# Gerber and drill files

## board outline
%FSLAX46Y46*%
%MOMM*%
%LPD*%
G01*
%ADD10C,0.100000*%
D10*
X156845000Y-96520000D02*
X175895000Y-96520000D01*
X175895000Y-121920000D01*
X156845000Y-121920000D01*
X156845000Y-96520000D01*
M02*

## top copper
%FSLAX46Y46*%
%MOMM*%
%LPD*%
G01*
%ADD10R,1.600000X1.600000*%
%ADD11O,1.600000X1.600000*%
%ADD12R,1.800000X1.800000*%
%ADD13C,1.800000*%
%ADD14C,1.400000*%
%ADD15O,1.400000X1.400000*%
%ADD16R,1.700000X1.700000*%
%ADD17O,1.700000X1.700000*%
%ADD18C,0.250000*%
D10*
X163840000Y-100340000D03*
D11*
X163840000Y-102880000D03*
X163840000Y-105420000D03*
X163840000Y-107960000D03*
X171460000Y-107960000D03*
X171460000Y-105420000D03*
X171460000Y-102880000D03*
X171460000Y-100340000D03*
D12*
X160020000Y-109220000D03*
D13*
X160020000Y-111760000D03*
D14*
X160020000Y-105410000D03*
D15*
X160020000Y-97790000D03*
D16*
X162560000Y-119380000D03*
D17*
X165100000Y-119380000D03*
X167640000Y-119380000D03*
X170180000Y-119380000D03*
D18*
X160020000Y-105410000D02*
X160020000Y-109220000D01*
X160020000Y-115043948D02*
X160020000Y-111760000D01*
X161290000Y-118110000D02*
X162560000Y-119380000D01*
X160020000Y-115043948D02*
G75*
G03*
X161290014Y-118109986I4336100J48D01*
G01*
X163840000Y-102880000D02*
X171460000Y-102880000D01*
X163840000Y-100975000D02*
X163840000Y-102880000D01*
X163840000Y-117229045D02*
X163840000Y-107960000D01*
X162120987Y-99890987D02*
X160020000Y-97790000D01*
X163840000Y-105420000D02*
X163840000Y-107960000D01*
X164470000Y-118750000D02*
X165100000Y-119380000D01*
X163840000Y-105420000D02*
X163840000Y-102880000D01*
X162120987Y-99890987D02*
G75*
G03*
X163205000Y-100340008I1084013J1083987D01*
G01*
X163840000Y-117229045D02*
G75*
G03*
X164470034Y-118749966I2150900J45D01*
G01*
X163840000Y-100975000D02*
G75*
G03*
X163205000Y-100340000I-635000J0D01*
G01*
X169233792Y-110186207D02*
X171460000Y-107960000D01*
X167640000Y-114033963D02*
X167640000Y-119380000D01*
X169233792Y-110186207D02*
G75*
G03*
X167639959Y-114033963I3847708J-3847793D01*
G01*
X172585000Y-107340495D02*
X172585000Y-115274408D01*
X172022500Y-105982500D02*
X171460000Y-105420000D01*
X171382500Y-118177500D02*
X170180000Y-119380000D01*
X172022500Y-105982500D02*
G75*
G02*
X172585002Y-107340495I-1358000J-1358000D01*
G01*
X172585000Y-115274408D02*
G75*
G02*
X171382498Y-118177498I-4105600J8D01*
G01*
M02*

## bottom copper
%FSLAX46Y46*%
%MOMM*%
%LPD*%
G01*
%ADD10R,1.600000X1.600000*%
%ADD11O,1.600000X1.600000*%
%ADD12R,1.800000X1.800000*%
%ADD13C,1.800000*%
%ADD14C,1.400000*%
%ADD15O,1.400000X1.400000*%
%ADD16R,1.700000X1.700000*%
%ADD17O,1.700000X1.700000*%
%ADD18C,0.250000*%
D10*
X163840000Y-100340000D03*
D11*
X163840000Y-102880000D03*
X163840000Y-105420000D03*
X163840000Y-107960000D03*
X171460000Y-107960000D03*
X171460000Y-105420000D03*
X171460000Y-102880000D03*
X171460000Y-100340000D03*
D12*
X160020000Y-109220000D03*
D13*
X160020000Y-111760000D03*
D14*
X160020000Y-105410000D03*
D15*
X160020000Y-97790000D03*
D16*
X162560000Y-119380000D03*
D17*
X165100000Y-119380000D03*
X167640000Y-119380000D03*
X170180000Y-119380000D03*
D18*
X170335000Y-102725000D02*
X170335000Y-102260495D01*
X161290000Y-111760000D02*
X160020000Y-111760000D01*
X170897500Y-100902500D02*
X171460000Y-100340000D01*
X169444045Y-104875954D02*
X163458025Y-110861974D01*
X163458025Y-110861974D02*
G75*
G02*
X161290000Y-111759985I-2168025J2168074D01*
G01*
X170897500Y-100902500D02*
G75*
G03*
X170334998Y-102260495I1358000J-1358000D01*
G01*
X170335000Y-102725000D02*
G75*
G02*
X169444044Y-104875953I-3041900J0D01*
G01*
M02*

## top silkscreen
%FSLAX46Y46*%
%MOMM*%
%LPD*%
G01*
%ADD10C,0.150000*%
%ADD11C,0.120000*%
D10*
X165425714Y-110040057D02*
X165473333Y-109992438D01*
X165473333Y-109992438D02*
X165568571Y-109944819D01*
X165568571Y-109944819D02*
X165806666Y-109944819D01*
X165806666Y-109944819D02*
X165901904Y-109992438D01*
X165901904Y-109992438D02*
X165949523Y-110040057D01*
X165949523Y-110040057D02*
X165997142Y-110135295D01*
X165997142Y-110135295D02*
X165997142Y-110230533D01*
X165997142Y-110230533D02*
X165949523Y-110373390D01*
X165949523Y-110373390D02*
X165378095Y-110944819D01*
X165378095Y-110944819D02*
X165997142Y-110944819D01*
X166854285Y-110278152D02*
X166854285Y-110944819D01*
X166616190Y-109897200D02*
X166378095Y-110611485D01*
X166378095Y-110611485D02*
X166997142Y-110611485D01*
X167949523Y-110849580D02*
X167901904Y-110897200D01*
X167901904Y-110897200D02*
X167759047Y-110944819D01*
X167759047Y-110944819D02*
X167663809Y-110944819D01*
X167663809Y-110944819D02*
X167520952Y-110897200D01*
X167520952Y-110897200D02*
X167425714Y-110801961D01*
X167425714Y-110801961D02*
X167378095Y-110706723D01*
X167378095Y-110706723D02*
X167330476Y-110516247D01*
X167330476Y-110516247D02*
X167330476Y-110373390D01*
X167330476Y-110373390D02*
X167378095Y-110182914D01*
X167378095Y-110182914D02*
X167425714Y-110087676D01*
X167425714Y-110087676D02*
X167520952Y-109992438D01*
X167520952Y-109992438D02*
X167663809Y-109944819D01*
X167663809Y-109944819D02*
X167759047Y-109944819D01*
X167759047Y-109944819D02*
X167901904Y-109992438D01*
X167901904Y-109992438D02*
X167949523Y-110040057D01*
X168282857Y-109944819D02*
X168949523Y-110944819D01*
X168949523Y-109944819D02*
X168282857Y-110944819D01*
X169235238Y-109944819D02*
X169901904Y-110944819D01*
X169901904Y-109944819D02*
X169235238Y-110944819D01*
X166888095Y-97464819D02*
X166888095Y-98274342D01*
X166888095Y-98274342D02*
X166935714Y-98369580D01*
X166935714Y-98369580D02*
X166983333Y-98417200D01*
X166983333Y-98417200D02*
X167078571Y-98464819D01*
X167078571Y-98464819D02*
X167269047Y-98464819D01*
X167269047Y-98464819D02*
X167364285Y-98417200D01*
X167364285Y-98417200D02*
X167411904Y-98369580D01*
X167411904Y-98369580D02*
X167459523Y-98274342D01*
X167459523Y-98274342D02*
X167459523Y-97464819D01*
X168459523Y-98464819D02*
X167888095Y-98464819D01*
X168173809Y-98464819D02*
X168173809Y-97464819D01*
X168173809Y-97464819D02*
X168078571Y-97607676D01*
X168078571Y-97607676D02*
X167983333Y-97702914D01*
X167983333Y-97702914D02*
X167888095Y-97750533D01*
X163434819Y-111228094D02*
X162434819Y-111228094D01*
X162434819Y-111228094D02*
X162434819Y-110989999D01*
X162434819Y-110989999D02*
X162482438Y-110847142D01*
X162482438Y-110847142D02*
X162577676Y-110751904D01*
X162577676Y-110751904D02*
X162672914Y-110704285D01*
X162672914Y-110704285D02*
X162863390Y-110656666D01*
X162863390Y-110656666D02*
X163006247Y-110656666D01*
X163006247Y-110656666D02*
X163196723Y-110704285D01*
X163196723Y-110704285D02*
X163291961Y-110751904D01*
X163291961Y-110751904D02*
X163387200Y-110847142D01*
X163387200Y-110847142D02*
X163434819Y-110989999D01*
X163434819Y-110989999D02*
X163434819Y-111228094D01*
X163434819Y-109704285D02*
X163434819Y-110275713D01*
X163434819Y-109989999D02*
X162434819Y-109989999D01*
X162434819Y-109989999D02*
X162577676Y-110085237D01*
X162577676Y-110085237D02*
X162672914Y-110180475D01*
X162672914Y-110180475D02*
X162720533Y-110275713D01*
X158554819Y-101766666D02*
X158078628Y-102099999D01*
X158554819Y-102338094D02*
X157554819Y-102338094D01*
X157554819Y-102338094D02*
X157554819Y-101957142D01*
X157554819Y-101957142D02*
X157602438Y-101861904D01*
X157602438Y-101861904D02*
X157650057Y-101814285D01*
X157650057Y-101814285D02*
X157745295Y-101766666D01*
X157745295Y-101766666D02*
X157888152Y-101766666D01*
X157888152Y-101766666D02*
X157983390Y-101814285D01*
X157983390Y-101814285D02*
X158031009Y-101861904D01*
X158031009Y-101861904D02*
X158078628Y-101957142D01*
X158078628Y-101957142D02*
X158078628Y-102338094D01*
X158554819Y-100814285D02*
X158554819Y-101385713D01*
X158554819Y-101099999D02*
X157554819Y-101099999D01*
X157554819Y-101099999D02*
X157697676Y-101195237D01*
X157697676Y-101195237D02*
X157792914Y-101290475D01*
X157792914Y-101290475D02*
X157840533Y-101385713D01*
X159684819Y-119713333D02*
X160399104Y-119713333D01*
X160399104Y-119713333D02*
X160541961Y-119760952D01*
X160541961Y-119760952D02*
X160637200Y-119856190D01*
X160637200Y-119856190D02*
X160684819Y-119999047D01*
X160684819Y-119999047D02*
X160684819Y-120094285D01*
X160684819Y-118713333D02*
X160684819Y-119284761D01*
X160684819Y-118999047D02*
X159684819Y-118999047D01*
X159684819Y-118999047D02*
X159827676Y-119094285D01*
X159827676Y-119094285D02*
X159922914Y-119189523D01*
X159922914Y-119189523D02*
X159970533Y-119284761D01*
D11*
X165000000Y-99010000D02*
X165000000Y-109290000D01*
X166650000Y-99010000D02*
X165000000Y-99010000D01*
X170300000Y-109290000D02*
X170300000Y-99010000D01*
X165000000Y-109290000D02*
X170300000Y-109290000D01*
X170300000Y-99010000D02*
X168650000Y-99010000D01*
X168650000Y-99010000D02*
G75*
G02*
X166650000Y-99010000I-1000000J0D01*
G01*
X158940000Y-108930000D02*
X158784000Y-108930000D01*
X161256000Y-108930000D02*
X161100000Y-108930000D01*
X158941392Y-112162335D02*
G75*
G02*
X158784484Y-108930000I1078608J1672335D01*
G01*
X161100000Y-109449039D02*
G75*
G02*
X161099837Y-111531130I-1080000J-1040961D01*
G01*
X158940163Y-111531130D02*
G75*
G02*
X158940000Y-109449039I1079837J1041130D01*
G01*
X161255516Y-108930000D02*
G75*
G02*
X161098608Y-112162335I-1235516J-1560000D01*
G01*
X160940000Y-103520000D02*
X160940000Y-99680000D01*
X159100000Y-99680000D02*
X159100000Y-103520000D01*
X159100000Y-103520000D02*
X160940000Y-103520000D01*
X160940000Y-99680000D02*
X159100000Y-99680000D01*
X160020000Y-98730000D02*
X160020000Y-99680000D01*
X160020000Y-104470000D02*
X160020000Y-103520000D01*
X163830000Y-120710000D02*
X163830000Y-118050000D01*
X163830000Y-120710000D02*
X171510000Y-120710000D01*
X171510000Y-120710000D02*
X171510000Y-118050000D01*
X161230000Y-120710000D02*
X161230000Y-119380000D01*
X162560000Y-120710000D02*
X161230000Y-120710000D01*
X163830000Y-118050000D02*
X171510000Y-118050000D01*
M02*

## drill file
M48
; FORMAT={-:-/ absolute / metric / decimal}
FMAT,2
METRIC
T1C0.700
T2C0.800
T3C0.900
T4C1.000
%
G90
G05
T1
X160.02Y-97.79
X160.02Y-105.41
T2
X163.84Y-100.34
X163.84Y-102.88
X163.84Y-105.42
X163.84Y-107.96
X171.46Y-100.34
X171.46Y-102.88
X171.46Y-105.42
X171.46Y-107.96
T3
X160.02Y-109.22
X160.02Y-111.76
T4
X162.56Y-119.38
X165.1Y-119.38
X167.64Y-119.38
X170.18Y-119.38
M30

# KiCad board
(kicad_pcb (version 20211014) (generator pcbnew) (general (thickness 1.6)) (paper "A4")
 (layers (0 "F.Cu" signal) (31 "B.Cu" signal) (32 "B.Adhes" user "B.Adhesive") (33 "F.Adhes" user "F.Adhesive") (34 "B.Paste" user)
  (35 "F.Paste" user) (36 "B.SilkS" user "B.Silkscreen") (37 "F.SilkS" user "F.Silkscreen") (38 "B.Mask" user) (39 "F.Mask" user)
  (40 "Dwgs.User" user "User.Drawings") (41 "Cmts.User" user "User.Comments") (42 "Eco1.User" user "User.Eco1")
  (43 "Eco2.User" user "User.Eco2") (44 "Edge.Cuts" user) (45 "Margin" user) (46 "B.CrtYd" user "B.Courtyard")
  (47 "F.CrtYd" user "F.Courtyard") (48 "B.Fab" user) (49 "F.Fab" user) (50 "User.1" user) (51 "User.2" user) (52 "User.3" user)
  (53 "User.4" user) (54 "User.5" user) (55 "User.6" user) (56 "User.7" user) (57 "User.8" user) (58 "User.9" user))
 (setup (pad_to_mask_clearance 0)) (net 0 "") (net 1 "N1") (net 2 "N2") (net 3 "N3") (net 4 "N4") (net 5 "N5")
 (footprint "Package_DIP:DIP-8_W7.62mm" (layer "F.Cu") (at 163.84 100.34)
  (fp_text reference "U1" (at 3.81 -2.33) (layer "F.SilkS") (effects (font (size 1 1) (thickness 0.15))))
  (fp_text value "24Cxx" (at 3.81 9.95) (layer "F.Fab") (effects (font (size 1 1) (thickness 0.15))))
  (fp_line (start 1.16 -1.33) (end 1.16 8.95) (layer "F.SilkS") (width 0.12))
  (fp_line (start 2.81 -1.33) (end 1.16 -1.33) (layer "F.SilkS") (width 0.12))
  (fp_line (start 6.46 8.95) (end 6.46 -1.33) (layer "F.SilkS") (width 0.12))
  (fp_line (start 1.16 8.95) (end 6.46 8.95) (layer "F.SilkS") (width 0.12))
  (fp_line (start 6.46 -1.33) (end 4.81 -1.33) (layer "F.SilkS") (width 0.12))
  (fp_arc (start 4.81 -1.33) (mid 3.81 -0.33) (end 2.81 -1.33) (layer "F.SilkS") (width 0.12))
  (pad "1" thru_hole rect (at 0 0) (size 1.6 1.6) (drill 0.8) (layers *.Cu *.Mask) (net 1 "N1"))
  (pad "2" thru_hole oval (at 0 2.54) (size 1.6 1.6) (drill 0.8) (layers *.Cu *.Mask) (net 1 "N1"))
  (pad "3" thru_hole oval (at 0 5.08) (size 1.6 1.6) (drill 0.8) (layers *.Cu *.Mask) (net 1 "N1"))
  (pad "4" thru_hole oval (at 0 7.62) (size 1.6 1.6) (drill 0.8) (layers *.Cu *.Mask) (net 1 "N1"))
  (pad "5" thru_hole oval (at 7.62 7.62) (size 1.6 1.6) (drill 0.8) (layers *.Cu *.Mask) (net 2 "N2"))
  (pad "6" thru_hole oval (at 7.62 5.08) (size 1.6 1.6) (drill 0.8) (layers *.Cu *.Mask) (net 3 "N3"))
  (pad "7" thru_hole oval (at 7.62 2.54) (size 1.6 1.6) (drill 0.8) (layers *.Cu *.Mask) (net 1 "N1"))
  (pad "8" thru_hole oval (at 7.62 0) (size 1.6 1.6) (drill 0.8) (layers *.Cu *.Mask) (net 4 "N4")))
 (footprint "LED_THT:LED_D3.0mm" (layer "F.Cu") (at 160.02 109.22 -90)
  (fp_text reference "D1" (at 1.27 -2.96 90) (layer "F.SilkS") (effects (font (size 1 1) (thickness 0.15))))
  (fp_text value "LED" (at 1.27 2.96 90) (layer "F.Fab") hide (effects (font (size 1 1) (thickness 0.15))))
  (fp_line (start -0.29 1.08) (end -0.29 1.236) (layer "F.SilkS") (width 0.12))
  (fp_line (start -0.29 -1.236) (end -0.29 -1.08) (layer "F.SilkS") (width 0.12))
  (fp_arc (start 2.942335 1.078608) (mid 1.366487 1.987659) (end -0.29 1.235516) (layer "F.SilkS") (width 0.12))
  (fp_arc (start 0.229039 -1.08) (mid 1.270117 -1.5) (end 2.31113 -1.079837) (layer "F.SilkS") (width 0.12))
  (fp_arc (start 2.31113 1.079837) (mid 1.270117 1.5) (end 0.229039 1.08) (layer "F.SilkS") (width 0.12))
  (fp_arc (start -0.29 -1.235516) (mid 1.366487 -1.987659) (end 2.942335 -1.078608) (layer "F.SilkS") (width 0.12))
  (pad "1" thru_hole rect (at 0 0 270) (size 1.8 1.8) (drill 0.9) (layers *.Cu *.Mask) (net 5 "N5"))
  (pad "2" thru_hole circle (at 2.54 0 270) (size 1.8 1.8) (drill 0.9) (layers *.Cu *.Mask) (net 4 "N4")))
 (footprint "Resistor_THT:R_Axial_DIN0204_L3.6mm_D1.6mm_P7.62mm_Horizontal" (layer "F.Cu") (at 160.02 105.41 90)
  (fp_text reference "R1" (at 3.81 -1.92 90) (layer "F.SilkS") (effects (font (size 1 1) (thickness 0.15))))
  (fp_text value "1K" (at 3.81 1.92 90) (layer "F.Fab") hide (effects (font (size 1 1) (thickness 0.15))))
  (fp_line (start 1.89 0.92) (end 5.73 0.92) (layer "F.SilkS") (width 0.12))
  (fp_line (start 5.73 -0.92) (end 1.89 -0.92) (layer "F.SilkS") (width 0.12))
  (fp_line (start 1.89 -0.92) (end 1.89 0.92) (layer "F.SilkS") (width 0.12))
  (fp_line (start 5.73 0.92) (end 5.73 -0.92) (layer "F.SilkS") (width 0.12))
  (fp_line (start 6.68 0) (end 5.73 0) (layer "F.SilkS") (width 0.12))
  (fp_line (start 0.94 0) (end 1.89 0) (layer "F.SilkS") (width 0.12))
  (pad "1" thru_hole circle (at 0 0 90) (size 1.4 1.4) (drill 0.7) (layers *.Cu *.Mask) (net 5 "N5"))
  (pad "2" thru_hole oval (at 7.62 0 90) (size 1.4 1.4) (drill 0.7) (layers *.Cu *.Mask) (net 1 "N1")))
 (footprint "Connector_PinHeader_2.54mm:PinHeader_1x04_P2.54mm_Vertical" (layer "F.Cu") (at 162.56 119.38 90)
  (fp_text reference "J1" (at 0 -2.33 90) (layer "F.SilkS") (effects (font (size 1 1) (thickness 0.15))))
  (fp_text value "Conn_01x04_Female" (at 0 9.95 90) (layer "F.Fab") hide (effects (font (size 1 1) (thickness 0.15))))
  (fp_line (start -1.33 1.27) (end 1.33 1.27) (layer "F.SilkS") (width 0.12))
  (fp_line (start -1.33 1.27) (end -1.33 8.95) (layer "F.SilkS") (width 0.12))
  (fp_line (start -1.33 8.95) (end 1.33 8.95) (layer "F.SilkS") (width 0.12))
  (fp_line (start -1.33 -1.33) (end 0 -1.33) (layer "F.SilkS") (width 0.12))
  (fp_line (start -1.33 0) (end -1.33 -1.33) (layer "F.SilkS") (width 0.12))
  (fp_line (start 1.33 1.27) (end 1.33 8.95) (layer "F.SilkS") (width 0.12))
  (pad "1" thru_hole rect (at 0 0 90) (size 1.7 1.7) (drill 1) (layers *.Cu *.Mask) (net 4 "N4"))
  (pad "2" thru_hole oval (at 0 2.54 90) (size 1.7 1.7) (drill 1) (layers *.Cu *.Mask) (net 1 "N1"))
  (pad "3" thru_hole oval (at 0 5.08 90) (size 1.7 1.7) (drill 1) (layers *.Cu *.Mask) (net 2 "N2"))
  (pad "4" thru_hole oval (at 0 7.62 90) (size 1.7 1.7) (drill 1) (layers *.Cu *.Mask) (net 3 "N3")))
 (gr_rect (start 156.845 96.52) (end 175.895 121.92) (layer "Edge.Cuts") (width 0.1) (fill none))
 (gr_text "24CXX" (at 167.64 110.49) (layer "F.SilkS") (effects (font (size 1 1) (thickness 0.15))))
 (segment (start 160.02 105.41) (end 160.02 109.22) (width 0.25) (layer "F.Cu") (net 5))
 (segment (start 160.02 115.043948) (end 160.02 111.76) (width 0.25) (layer "F.Cu") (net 4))
 (segment (start 161.29 118.11) (end 162.56 119.38) (width 0.25) (layer "F.Cu") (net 4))
 (arc (start 160.02 115.043948) (mid 160.350062 116.703283) (end 161.29 118.11) (width 0.25) (layer "F.Cu") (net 4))
 (segment (start 170.335 102.725) (end 170.335 102.260495) (width 0.25) (layer "B.Cu") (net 4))
 (segment (start 161.29 111.76) (end 160.02 111.76) (width 0.25) (layer "B.Cu") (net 4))
 (segment (start 170.8975 100.9025) (end 171.46 100.34) (width 0.25) (layer "B.Cu") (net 4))
 (segment (start 169.444045 104.875954) (end 163.458025 110.861974) (width 0.25) (layer "B.Cu") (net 4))
 (arc (start 163.458025 110.861974) (mid 162.463326 111.52661) (end 161.29 111.76) (width 0.25) (layer "B.Cu") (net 4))
 (arc (start 170.8975 100.9025) (mid 170.481188 101.525553) (end 170.335 102.260495) (width 0.25) (layer "B.Cu") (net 4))
 (arc (start 170.335 102.725) (mid 170.103448 103.889088) (end 169.444045 104.875954) (width 0.25) (layer "B.Cu") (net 4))
 (segment (start 163.84 102.88) (end 171.46 102.88) (width 0.25) (layer "F.Cu") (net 1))
 (segment (start 163.84 100.975) (end 163.84 102.88) (width 0.25) (layer "F.Cu") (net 1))
 (segment (start 163.84 117.229045) (end 163.84 107.96) (width 0.25) (layer "F.Cu") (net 1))
 (segment (start 162.120987 99.890987) (end 160.02 97.79) (width 0.25) (layer "F.Cu") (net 1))
 (segment (start 163.84 105.42) (end 163.84 107.96) (width 0.25) (layer "F.Cu") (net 1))
 (segment (start 164.47 118.75) (end 165.1 119.38) (width 0.25) (layer "F.Cu") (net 1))
 (segment (start 163.84 105.42) (end 163.84 102.88) (width 0.25) (layer "F.Cu") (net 1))
 (arc (start 162.120987 99.890987) (mid 162.618336 100.223305) (end 163.205 100.34) (width 0.25) (layer "F.Cu") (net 1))
 (arc (start 163.84 117.229045) (mid 164.003731 118.05218) (end 164.47 118.75) (width 0.25) (layer "F.Cu") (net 1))
 (arc (start 163.84 100.975) (mid 163.654012 100.525987) (end 163.205 100.34) (width 0.25) (layer "F.Cu") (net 1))
 (segment (start 169.233792 110.186207) (end 171.46 107.96) (width 0.25) (layer "F.Cu") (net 2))
 (segment (start 167.64 114.033963) (end 167.64 119.38) (width 0.25) (layer "F.Cu") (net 2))
 (arc (start 169.233792 110.186207) (mid 168.054213 111.951572) (end 167.64 114.033963) (width 0.25) (layer "F.Cu") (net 2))
 (segment (start 172.585 107.340495) (end 172.585 115.274408) (width 0.25) (layer "F.Cu") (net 3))
 (segment (start 172.0225 105.9825) (end 171.46 105.42) (width 0.25) (layer "F.Cu") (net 3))
 (segment (start 171.3825 118.1775) (end 170.18 119.38) (width 0.25) (layer "F.Cu") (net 3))
 (arc (start 172.0225 105.9825) (mid 172.438811 106.605553) (end 172.585 107.340495) (width 0.25) (layer "F.Cu") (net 3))
 (arc (start 172.585 115.274408) (mid 172.27248 116.84555) (end 171.3825 118.1775) (width 0.25) (layer "F.Cu") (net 3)))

